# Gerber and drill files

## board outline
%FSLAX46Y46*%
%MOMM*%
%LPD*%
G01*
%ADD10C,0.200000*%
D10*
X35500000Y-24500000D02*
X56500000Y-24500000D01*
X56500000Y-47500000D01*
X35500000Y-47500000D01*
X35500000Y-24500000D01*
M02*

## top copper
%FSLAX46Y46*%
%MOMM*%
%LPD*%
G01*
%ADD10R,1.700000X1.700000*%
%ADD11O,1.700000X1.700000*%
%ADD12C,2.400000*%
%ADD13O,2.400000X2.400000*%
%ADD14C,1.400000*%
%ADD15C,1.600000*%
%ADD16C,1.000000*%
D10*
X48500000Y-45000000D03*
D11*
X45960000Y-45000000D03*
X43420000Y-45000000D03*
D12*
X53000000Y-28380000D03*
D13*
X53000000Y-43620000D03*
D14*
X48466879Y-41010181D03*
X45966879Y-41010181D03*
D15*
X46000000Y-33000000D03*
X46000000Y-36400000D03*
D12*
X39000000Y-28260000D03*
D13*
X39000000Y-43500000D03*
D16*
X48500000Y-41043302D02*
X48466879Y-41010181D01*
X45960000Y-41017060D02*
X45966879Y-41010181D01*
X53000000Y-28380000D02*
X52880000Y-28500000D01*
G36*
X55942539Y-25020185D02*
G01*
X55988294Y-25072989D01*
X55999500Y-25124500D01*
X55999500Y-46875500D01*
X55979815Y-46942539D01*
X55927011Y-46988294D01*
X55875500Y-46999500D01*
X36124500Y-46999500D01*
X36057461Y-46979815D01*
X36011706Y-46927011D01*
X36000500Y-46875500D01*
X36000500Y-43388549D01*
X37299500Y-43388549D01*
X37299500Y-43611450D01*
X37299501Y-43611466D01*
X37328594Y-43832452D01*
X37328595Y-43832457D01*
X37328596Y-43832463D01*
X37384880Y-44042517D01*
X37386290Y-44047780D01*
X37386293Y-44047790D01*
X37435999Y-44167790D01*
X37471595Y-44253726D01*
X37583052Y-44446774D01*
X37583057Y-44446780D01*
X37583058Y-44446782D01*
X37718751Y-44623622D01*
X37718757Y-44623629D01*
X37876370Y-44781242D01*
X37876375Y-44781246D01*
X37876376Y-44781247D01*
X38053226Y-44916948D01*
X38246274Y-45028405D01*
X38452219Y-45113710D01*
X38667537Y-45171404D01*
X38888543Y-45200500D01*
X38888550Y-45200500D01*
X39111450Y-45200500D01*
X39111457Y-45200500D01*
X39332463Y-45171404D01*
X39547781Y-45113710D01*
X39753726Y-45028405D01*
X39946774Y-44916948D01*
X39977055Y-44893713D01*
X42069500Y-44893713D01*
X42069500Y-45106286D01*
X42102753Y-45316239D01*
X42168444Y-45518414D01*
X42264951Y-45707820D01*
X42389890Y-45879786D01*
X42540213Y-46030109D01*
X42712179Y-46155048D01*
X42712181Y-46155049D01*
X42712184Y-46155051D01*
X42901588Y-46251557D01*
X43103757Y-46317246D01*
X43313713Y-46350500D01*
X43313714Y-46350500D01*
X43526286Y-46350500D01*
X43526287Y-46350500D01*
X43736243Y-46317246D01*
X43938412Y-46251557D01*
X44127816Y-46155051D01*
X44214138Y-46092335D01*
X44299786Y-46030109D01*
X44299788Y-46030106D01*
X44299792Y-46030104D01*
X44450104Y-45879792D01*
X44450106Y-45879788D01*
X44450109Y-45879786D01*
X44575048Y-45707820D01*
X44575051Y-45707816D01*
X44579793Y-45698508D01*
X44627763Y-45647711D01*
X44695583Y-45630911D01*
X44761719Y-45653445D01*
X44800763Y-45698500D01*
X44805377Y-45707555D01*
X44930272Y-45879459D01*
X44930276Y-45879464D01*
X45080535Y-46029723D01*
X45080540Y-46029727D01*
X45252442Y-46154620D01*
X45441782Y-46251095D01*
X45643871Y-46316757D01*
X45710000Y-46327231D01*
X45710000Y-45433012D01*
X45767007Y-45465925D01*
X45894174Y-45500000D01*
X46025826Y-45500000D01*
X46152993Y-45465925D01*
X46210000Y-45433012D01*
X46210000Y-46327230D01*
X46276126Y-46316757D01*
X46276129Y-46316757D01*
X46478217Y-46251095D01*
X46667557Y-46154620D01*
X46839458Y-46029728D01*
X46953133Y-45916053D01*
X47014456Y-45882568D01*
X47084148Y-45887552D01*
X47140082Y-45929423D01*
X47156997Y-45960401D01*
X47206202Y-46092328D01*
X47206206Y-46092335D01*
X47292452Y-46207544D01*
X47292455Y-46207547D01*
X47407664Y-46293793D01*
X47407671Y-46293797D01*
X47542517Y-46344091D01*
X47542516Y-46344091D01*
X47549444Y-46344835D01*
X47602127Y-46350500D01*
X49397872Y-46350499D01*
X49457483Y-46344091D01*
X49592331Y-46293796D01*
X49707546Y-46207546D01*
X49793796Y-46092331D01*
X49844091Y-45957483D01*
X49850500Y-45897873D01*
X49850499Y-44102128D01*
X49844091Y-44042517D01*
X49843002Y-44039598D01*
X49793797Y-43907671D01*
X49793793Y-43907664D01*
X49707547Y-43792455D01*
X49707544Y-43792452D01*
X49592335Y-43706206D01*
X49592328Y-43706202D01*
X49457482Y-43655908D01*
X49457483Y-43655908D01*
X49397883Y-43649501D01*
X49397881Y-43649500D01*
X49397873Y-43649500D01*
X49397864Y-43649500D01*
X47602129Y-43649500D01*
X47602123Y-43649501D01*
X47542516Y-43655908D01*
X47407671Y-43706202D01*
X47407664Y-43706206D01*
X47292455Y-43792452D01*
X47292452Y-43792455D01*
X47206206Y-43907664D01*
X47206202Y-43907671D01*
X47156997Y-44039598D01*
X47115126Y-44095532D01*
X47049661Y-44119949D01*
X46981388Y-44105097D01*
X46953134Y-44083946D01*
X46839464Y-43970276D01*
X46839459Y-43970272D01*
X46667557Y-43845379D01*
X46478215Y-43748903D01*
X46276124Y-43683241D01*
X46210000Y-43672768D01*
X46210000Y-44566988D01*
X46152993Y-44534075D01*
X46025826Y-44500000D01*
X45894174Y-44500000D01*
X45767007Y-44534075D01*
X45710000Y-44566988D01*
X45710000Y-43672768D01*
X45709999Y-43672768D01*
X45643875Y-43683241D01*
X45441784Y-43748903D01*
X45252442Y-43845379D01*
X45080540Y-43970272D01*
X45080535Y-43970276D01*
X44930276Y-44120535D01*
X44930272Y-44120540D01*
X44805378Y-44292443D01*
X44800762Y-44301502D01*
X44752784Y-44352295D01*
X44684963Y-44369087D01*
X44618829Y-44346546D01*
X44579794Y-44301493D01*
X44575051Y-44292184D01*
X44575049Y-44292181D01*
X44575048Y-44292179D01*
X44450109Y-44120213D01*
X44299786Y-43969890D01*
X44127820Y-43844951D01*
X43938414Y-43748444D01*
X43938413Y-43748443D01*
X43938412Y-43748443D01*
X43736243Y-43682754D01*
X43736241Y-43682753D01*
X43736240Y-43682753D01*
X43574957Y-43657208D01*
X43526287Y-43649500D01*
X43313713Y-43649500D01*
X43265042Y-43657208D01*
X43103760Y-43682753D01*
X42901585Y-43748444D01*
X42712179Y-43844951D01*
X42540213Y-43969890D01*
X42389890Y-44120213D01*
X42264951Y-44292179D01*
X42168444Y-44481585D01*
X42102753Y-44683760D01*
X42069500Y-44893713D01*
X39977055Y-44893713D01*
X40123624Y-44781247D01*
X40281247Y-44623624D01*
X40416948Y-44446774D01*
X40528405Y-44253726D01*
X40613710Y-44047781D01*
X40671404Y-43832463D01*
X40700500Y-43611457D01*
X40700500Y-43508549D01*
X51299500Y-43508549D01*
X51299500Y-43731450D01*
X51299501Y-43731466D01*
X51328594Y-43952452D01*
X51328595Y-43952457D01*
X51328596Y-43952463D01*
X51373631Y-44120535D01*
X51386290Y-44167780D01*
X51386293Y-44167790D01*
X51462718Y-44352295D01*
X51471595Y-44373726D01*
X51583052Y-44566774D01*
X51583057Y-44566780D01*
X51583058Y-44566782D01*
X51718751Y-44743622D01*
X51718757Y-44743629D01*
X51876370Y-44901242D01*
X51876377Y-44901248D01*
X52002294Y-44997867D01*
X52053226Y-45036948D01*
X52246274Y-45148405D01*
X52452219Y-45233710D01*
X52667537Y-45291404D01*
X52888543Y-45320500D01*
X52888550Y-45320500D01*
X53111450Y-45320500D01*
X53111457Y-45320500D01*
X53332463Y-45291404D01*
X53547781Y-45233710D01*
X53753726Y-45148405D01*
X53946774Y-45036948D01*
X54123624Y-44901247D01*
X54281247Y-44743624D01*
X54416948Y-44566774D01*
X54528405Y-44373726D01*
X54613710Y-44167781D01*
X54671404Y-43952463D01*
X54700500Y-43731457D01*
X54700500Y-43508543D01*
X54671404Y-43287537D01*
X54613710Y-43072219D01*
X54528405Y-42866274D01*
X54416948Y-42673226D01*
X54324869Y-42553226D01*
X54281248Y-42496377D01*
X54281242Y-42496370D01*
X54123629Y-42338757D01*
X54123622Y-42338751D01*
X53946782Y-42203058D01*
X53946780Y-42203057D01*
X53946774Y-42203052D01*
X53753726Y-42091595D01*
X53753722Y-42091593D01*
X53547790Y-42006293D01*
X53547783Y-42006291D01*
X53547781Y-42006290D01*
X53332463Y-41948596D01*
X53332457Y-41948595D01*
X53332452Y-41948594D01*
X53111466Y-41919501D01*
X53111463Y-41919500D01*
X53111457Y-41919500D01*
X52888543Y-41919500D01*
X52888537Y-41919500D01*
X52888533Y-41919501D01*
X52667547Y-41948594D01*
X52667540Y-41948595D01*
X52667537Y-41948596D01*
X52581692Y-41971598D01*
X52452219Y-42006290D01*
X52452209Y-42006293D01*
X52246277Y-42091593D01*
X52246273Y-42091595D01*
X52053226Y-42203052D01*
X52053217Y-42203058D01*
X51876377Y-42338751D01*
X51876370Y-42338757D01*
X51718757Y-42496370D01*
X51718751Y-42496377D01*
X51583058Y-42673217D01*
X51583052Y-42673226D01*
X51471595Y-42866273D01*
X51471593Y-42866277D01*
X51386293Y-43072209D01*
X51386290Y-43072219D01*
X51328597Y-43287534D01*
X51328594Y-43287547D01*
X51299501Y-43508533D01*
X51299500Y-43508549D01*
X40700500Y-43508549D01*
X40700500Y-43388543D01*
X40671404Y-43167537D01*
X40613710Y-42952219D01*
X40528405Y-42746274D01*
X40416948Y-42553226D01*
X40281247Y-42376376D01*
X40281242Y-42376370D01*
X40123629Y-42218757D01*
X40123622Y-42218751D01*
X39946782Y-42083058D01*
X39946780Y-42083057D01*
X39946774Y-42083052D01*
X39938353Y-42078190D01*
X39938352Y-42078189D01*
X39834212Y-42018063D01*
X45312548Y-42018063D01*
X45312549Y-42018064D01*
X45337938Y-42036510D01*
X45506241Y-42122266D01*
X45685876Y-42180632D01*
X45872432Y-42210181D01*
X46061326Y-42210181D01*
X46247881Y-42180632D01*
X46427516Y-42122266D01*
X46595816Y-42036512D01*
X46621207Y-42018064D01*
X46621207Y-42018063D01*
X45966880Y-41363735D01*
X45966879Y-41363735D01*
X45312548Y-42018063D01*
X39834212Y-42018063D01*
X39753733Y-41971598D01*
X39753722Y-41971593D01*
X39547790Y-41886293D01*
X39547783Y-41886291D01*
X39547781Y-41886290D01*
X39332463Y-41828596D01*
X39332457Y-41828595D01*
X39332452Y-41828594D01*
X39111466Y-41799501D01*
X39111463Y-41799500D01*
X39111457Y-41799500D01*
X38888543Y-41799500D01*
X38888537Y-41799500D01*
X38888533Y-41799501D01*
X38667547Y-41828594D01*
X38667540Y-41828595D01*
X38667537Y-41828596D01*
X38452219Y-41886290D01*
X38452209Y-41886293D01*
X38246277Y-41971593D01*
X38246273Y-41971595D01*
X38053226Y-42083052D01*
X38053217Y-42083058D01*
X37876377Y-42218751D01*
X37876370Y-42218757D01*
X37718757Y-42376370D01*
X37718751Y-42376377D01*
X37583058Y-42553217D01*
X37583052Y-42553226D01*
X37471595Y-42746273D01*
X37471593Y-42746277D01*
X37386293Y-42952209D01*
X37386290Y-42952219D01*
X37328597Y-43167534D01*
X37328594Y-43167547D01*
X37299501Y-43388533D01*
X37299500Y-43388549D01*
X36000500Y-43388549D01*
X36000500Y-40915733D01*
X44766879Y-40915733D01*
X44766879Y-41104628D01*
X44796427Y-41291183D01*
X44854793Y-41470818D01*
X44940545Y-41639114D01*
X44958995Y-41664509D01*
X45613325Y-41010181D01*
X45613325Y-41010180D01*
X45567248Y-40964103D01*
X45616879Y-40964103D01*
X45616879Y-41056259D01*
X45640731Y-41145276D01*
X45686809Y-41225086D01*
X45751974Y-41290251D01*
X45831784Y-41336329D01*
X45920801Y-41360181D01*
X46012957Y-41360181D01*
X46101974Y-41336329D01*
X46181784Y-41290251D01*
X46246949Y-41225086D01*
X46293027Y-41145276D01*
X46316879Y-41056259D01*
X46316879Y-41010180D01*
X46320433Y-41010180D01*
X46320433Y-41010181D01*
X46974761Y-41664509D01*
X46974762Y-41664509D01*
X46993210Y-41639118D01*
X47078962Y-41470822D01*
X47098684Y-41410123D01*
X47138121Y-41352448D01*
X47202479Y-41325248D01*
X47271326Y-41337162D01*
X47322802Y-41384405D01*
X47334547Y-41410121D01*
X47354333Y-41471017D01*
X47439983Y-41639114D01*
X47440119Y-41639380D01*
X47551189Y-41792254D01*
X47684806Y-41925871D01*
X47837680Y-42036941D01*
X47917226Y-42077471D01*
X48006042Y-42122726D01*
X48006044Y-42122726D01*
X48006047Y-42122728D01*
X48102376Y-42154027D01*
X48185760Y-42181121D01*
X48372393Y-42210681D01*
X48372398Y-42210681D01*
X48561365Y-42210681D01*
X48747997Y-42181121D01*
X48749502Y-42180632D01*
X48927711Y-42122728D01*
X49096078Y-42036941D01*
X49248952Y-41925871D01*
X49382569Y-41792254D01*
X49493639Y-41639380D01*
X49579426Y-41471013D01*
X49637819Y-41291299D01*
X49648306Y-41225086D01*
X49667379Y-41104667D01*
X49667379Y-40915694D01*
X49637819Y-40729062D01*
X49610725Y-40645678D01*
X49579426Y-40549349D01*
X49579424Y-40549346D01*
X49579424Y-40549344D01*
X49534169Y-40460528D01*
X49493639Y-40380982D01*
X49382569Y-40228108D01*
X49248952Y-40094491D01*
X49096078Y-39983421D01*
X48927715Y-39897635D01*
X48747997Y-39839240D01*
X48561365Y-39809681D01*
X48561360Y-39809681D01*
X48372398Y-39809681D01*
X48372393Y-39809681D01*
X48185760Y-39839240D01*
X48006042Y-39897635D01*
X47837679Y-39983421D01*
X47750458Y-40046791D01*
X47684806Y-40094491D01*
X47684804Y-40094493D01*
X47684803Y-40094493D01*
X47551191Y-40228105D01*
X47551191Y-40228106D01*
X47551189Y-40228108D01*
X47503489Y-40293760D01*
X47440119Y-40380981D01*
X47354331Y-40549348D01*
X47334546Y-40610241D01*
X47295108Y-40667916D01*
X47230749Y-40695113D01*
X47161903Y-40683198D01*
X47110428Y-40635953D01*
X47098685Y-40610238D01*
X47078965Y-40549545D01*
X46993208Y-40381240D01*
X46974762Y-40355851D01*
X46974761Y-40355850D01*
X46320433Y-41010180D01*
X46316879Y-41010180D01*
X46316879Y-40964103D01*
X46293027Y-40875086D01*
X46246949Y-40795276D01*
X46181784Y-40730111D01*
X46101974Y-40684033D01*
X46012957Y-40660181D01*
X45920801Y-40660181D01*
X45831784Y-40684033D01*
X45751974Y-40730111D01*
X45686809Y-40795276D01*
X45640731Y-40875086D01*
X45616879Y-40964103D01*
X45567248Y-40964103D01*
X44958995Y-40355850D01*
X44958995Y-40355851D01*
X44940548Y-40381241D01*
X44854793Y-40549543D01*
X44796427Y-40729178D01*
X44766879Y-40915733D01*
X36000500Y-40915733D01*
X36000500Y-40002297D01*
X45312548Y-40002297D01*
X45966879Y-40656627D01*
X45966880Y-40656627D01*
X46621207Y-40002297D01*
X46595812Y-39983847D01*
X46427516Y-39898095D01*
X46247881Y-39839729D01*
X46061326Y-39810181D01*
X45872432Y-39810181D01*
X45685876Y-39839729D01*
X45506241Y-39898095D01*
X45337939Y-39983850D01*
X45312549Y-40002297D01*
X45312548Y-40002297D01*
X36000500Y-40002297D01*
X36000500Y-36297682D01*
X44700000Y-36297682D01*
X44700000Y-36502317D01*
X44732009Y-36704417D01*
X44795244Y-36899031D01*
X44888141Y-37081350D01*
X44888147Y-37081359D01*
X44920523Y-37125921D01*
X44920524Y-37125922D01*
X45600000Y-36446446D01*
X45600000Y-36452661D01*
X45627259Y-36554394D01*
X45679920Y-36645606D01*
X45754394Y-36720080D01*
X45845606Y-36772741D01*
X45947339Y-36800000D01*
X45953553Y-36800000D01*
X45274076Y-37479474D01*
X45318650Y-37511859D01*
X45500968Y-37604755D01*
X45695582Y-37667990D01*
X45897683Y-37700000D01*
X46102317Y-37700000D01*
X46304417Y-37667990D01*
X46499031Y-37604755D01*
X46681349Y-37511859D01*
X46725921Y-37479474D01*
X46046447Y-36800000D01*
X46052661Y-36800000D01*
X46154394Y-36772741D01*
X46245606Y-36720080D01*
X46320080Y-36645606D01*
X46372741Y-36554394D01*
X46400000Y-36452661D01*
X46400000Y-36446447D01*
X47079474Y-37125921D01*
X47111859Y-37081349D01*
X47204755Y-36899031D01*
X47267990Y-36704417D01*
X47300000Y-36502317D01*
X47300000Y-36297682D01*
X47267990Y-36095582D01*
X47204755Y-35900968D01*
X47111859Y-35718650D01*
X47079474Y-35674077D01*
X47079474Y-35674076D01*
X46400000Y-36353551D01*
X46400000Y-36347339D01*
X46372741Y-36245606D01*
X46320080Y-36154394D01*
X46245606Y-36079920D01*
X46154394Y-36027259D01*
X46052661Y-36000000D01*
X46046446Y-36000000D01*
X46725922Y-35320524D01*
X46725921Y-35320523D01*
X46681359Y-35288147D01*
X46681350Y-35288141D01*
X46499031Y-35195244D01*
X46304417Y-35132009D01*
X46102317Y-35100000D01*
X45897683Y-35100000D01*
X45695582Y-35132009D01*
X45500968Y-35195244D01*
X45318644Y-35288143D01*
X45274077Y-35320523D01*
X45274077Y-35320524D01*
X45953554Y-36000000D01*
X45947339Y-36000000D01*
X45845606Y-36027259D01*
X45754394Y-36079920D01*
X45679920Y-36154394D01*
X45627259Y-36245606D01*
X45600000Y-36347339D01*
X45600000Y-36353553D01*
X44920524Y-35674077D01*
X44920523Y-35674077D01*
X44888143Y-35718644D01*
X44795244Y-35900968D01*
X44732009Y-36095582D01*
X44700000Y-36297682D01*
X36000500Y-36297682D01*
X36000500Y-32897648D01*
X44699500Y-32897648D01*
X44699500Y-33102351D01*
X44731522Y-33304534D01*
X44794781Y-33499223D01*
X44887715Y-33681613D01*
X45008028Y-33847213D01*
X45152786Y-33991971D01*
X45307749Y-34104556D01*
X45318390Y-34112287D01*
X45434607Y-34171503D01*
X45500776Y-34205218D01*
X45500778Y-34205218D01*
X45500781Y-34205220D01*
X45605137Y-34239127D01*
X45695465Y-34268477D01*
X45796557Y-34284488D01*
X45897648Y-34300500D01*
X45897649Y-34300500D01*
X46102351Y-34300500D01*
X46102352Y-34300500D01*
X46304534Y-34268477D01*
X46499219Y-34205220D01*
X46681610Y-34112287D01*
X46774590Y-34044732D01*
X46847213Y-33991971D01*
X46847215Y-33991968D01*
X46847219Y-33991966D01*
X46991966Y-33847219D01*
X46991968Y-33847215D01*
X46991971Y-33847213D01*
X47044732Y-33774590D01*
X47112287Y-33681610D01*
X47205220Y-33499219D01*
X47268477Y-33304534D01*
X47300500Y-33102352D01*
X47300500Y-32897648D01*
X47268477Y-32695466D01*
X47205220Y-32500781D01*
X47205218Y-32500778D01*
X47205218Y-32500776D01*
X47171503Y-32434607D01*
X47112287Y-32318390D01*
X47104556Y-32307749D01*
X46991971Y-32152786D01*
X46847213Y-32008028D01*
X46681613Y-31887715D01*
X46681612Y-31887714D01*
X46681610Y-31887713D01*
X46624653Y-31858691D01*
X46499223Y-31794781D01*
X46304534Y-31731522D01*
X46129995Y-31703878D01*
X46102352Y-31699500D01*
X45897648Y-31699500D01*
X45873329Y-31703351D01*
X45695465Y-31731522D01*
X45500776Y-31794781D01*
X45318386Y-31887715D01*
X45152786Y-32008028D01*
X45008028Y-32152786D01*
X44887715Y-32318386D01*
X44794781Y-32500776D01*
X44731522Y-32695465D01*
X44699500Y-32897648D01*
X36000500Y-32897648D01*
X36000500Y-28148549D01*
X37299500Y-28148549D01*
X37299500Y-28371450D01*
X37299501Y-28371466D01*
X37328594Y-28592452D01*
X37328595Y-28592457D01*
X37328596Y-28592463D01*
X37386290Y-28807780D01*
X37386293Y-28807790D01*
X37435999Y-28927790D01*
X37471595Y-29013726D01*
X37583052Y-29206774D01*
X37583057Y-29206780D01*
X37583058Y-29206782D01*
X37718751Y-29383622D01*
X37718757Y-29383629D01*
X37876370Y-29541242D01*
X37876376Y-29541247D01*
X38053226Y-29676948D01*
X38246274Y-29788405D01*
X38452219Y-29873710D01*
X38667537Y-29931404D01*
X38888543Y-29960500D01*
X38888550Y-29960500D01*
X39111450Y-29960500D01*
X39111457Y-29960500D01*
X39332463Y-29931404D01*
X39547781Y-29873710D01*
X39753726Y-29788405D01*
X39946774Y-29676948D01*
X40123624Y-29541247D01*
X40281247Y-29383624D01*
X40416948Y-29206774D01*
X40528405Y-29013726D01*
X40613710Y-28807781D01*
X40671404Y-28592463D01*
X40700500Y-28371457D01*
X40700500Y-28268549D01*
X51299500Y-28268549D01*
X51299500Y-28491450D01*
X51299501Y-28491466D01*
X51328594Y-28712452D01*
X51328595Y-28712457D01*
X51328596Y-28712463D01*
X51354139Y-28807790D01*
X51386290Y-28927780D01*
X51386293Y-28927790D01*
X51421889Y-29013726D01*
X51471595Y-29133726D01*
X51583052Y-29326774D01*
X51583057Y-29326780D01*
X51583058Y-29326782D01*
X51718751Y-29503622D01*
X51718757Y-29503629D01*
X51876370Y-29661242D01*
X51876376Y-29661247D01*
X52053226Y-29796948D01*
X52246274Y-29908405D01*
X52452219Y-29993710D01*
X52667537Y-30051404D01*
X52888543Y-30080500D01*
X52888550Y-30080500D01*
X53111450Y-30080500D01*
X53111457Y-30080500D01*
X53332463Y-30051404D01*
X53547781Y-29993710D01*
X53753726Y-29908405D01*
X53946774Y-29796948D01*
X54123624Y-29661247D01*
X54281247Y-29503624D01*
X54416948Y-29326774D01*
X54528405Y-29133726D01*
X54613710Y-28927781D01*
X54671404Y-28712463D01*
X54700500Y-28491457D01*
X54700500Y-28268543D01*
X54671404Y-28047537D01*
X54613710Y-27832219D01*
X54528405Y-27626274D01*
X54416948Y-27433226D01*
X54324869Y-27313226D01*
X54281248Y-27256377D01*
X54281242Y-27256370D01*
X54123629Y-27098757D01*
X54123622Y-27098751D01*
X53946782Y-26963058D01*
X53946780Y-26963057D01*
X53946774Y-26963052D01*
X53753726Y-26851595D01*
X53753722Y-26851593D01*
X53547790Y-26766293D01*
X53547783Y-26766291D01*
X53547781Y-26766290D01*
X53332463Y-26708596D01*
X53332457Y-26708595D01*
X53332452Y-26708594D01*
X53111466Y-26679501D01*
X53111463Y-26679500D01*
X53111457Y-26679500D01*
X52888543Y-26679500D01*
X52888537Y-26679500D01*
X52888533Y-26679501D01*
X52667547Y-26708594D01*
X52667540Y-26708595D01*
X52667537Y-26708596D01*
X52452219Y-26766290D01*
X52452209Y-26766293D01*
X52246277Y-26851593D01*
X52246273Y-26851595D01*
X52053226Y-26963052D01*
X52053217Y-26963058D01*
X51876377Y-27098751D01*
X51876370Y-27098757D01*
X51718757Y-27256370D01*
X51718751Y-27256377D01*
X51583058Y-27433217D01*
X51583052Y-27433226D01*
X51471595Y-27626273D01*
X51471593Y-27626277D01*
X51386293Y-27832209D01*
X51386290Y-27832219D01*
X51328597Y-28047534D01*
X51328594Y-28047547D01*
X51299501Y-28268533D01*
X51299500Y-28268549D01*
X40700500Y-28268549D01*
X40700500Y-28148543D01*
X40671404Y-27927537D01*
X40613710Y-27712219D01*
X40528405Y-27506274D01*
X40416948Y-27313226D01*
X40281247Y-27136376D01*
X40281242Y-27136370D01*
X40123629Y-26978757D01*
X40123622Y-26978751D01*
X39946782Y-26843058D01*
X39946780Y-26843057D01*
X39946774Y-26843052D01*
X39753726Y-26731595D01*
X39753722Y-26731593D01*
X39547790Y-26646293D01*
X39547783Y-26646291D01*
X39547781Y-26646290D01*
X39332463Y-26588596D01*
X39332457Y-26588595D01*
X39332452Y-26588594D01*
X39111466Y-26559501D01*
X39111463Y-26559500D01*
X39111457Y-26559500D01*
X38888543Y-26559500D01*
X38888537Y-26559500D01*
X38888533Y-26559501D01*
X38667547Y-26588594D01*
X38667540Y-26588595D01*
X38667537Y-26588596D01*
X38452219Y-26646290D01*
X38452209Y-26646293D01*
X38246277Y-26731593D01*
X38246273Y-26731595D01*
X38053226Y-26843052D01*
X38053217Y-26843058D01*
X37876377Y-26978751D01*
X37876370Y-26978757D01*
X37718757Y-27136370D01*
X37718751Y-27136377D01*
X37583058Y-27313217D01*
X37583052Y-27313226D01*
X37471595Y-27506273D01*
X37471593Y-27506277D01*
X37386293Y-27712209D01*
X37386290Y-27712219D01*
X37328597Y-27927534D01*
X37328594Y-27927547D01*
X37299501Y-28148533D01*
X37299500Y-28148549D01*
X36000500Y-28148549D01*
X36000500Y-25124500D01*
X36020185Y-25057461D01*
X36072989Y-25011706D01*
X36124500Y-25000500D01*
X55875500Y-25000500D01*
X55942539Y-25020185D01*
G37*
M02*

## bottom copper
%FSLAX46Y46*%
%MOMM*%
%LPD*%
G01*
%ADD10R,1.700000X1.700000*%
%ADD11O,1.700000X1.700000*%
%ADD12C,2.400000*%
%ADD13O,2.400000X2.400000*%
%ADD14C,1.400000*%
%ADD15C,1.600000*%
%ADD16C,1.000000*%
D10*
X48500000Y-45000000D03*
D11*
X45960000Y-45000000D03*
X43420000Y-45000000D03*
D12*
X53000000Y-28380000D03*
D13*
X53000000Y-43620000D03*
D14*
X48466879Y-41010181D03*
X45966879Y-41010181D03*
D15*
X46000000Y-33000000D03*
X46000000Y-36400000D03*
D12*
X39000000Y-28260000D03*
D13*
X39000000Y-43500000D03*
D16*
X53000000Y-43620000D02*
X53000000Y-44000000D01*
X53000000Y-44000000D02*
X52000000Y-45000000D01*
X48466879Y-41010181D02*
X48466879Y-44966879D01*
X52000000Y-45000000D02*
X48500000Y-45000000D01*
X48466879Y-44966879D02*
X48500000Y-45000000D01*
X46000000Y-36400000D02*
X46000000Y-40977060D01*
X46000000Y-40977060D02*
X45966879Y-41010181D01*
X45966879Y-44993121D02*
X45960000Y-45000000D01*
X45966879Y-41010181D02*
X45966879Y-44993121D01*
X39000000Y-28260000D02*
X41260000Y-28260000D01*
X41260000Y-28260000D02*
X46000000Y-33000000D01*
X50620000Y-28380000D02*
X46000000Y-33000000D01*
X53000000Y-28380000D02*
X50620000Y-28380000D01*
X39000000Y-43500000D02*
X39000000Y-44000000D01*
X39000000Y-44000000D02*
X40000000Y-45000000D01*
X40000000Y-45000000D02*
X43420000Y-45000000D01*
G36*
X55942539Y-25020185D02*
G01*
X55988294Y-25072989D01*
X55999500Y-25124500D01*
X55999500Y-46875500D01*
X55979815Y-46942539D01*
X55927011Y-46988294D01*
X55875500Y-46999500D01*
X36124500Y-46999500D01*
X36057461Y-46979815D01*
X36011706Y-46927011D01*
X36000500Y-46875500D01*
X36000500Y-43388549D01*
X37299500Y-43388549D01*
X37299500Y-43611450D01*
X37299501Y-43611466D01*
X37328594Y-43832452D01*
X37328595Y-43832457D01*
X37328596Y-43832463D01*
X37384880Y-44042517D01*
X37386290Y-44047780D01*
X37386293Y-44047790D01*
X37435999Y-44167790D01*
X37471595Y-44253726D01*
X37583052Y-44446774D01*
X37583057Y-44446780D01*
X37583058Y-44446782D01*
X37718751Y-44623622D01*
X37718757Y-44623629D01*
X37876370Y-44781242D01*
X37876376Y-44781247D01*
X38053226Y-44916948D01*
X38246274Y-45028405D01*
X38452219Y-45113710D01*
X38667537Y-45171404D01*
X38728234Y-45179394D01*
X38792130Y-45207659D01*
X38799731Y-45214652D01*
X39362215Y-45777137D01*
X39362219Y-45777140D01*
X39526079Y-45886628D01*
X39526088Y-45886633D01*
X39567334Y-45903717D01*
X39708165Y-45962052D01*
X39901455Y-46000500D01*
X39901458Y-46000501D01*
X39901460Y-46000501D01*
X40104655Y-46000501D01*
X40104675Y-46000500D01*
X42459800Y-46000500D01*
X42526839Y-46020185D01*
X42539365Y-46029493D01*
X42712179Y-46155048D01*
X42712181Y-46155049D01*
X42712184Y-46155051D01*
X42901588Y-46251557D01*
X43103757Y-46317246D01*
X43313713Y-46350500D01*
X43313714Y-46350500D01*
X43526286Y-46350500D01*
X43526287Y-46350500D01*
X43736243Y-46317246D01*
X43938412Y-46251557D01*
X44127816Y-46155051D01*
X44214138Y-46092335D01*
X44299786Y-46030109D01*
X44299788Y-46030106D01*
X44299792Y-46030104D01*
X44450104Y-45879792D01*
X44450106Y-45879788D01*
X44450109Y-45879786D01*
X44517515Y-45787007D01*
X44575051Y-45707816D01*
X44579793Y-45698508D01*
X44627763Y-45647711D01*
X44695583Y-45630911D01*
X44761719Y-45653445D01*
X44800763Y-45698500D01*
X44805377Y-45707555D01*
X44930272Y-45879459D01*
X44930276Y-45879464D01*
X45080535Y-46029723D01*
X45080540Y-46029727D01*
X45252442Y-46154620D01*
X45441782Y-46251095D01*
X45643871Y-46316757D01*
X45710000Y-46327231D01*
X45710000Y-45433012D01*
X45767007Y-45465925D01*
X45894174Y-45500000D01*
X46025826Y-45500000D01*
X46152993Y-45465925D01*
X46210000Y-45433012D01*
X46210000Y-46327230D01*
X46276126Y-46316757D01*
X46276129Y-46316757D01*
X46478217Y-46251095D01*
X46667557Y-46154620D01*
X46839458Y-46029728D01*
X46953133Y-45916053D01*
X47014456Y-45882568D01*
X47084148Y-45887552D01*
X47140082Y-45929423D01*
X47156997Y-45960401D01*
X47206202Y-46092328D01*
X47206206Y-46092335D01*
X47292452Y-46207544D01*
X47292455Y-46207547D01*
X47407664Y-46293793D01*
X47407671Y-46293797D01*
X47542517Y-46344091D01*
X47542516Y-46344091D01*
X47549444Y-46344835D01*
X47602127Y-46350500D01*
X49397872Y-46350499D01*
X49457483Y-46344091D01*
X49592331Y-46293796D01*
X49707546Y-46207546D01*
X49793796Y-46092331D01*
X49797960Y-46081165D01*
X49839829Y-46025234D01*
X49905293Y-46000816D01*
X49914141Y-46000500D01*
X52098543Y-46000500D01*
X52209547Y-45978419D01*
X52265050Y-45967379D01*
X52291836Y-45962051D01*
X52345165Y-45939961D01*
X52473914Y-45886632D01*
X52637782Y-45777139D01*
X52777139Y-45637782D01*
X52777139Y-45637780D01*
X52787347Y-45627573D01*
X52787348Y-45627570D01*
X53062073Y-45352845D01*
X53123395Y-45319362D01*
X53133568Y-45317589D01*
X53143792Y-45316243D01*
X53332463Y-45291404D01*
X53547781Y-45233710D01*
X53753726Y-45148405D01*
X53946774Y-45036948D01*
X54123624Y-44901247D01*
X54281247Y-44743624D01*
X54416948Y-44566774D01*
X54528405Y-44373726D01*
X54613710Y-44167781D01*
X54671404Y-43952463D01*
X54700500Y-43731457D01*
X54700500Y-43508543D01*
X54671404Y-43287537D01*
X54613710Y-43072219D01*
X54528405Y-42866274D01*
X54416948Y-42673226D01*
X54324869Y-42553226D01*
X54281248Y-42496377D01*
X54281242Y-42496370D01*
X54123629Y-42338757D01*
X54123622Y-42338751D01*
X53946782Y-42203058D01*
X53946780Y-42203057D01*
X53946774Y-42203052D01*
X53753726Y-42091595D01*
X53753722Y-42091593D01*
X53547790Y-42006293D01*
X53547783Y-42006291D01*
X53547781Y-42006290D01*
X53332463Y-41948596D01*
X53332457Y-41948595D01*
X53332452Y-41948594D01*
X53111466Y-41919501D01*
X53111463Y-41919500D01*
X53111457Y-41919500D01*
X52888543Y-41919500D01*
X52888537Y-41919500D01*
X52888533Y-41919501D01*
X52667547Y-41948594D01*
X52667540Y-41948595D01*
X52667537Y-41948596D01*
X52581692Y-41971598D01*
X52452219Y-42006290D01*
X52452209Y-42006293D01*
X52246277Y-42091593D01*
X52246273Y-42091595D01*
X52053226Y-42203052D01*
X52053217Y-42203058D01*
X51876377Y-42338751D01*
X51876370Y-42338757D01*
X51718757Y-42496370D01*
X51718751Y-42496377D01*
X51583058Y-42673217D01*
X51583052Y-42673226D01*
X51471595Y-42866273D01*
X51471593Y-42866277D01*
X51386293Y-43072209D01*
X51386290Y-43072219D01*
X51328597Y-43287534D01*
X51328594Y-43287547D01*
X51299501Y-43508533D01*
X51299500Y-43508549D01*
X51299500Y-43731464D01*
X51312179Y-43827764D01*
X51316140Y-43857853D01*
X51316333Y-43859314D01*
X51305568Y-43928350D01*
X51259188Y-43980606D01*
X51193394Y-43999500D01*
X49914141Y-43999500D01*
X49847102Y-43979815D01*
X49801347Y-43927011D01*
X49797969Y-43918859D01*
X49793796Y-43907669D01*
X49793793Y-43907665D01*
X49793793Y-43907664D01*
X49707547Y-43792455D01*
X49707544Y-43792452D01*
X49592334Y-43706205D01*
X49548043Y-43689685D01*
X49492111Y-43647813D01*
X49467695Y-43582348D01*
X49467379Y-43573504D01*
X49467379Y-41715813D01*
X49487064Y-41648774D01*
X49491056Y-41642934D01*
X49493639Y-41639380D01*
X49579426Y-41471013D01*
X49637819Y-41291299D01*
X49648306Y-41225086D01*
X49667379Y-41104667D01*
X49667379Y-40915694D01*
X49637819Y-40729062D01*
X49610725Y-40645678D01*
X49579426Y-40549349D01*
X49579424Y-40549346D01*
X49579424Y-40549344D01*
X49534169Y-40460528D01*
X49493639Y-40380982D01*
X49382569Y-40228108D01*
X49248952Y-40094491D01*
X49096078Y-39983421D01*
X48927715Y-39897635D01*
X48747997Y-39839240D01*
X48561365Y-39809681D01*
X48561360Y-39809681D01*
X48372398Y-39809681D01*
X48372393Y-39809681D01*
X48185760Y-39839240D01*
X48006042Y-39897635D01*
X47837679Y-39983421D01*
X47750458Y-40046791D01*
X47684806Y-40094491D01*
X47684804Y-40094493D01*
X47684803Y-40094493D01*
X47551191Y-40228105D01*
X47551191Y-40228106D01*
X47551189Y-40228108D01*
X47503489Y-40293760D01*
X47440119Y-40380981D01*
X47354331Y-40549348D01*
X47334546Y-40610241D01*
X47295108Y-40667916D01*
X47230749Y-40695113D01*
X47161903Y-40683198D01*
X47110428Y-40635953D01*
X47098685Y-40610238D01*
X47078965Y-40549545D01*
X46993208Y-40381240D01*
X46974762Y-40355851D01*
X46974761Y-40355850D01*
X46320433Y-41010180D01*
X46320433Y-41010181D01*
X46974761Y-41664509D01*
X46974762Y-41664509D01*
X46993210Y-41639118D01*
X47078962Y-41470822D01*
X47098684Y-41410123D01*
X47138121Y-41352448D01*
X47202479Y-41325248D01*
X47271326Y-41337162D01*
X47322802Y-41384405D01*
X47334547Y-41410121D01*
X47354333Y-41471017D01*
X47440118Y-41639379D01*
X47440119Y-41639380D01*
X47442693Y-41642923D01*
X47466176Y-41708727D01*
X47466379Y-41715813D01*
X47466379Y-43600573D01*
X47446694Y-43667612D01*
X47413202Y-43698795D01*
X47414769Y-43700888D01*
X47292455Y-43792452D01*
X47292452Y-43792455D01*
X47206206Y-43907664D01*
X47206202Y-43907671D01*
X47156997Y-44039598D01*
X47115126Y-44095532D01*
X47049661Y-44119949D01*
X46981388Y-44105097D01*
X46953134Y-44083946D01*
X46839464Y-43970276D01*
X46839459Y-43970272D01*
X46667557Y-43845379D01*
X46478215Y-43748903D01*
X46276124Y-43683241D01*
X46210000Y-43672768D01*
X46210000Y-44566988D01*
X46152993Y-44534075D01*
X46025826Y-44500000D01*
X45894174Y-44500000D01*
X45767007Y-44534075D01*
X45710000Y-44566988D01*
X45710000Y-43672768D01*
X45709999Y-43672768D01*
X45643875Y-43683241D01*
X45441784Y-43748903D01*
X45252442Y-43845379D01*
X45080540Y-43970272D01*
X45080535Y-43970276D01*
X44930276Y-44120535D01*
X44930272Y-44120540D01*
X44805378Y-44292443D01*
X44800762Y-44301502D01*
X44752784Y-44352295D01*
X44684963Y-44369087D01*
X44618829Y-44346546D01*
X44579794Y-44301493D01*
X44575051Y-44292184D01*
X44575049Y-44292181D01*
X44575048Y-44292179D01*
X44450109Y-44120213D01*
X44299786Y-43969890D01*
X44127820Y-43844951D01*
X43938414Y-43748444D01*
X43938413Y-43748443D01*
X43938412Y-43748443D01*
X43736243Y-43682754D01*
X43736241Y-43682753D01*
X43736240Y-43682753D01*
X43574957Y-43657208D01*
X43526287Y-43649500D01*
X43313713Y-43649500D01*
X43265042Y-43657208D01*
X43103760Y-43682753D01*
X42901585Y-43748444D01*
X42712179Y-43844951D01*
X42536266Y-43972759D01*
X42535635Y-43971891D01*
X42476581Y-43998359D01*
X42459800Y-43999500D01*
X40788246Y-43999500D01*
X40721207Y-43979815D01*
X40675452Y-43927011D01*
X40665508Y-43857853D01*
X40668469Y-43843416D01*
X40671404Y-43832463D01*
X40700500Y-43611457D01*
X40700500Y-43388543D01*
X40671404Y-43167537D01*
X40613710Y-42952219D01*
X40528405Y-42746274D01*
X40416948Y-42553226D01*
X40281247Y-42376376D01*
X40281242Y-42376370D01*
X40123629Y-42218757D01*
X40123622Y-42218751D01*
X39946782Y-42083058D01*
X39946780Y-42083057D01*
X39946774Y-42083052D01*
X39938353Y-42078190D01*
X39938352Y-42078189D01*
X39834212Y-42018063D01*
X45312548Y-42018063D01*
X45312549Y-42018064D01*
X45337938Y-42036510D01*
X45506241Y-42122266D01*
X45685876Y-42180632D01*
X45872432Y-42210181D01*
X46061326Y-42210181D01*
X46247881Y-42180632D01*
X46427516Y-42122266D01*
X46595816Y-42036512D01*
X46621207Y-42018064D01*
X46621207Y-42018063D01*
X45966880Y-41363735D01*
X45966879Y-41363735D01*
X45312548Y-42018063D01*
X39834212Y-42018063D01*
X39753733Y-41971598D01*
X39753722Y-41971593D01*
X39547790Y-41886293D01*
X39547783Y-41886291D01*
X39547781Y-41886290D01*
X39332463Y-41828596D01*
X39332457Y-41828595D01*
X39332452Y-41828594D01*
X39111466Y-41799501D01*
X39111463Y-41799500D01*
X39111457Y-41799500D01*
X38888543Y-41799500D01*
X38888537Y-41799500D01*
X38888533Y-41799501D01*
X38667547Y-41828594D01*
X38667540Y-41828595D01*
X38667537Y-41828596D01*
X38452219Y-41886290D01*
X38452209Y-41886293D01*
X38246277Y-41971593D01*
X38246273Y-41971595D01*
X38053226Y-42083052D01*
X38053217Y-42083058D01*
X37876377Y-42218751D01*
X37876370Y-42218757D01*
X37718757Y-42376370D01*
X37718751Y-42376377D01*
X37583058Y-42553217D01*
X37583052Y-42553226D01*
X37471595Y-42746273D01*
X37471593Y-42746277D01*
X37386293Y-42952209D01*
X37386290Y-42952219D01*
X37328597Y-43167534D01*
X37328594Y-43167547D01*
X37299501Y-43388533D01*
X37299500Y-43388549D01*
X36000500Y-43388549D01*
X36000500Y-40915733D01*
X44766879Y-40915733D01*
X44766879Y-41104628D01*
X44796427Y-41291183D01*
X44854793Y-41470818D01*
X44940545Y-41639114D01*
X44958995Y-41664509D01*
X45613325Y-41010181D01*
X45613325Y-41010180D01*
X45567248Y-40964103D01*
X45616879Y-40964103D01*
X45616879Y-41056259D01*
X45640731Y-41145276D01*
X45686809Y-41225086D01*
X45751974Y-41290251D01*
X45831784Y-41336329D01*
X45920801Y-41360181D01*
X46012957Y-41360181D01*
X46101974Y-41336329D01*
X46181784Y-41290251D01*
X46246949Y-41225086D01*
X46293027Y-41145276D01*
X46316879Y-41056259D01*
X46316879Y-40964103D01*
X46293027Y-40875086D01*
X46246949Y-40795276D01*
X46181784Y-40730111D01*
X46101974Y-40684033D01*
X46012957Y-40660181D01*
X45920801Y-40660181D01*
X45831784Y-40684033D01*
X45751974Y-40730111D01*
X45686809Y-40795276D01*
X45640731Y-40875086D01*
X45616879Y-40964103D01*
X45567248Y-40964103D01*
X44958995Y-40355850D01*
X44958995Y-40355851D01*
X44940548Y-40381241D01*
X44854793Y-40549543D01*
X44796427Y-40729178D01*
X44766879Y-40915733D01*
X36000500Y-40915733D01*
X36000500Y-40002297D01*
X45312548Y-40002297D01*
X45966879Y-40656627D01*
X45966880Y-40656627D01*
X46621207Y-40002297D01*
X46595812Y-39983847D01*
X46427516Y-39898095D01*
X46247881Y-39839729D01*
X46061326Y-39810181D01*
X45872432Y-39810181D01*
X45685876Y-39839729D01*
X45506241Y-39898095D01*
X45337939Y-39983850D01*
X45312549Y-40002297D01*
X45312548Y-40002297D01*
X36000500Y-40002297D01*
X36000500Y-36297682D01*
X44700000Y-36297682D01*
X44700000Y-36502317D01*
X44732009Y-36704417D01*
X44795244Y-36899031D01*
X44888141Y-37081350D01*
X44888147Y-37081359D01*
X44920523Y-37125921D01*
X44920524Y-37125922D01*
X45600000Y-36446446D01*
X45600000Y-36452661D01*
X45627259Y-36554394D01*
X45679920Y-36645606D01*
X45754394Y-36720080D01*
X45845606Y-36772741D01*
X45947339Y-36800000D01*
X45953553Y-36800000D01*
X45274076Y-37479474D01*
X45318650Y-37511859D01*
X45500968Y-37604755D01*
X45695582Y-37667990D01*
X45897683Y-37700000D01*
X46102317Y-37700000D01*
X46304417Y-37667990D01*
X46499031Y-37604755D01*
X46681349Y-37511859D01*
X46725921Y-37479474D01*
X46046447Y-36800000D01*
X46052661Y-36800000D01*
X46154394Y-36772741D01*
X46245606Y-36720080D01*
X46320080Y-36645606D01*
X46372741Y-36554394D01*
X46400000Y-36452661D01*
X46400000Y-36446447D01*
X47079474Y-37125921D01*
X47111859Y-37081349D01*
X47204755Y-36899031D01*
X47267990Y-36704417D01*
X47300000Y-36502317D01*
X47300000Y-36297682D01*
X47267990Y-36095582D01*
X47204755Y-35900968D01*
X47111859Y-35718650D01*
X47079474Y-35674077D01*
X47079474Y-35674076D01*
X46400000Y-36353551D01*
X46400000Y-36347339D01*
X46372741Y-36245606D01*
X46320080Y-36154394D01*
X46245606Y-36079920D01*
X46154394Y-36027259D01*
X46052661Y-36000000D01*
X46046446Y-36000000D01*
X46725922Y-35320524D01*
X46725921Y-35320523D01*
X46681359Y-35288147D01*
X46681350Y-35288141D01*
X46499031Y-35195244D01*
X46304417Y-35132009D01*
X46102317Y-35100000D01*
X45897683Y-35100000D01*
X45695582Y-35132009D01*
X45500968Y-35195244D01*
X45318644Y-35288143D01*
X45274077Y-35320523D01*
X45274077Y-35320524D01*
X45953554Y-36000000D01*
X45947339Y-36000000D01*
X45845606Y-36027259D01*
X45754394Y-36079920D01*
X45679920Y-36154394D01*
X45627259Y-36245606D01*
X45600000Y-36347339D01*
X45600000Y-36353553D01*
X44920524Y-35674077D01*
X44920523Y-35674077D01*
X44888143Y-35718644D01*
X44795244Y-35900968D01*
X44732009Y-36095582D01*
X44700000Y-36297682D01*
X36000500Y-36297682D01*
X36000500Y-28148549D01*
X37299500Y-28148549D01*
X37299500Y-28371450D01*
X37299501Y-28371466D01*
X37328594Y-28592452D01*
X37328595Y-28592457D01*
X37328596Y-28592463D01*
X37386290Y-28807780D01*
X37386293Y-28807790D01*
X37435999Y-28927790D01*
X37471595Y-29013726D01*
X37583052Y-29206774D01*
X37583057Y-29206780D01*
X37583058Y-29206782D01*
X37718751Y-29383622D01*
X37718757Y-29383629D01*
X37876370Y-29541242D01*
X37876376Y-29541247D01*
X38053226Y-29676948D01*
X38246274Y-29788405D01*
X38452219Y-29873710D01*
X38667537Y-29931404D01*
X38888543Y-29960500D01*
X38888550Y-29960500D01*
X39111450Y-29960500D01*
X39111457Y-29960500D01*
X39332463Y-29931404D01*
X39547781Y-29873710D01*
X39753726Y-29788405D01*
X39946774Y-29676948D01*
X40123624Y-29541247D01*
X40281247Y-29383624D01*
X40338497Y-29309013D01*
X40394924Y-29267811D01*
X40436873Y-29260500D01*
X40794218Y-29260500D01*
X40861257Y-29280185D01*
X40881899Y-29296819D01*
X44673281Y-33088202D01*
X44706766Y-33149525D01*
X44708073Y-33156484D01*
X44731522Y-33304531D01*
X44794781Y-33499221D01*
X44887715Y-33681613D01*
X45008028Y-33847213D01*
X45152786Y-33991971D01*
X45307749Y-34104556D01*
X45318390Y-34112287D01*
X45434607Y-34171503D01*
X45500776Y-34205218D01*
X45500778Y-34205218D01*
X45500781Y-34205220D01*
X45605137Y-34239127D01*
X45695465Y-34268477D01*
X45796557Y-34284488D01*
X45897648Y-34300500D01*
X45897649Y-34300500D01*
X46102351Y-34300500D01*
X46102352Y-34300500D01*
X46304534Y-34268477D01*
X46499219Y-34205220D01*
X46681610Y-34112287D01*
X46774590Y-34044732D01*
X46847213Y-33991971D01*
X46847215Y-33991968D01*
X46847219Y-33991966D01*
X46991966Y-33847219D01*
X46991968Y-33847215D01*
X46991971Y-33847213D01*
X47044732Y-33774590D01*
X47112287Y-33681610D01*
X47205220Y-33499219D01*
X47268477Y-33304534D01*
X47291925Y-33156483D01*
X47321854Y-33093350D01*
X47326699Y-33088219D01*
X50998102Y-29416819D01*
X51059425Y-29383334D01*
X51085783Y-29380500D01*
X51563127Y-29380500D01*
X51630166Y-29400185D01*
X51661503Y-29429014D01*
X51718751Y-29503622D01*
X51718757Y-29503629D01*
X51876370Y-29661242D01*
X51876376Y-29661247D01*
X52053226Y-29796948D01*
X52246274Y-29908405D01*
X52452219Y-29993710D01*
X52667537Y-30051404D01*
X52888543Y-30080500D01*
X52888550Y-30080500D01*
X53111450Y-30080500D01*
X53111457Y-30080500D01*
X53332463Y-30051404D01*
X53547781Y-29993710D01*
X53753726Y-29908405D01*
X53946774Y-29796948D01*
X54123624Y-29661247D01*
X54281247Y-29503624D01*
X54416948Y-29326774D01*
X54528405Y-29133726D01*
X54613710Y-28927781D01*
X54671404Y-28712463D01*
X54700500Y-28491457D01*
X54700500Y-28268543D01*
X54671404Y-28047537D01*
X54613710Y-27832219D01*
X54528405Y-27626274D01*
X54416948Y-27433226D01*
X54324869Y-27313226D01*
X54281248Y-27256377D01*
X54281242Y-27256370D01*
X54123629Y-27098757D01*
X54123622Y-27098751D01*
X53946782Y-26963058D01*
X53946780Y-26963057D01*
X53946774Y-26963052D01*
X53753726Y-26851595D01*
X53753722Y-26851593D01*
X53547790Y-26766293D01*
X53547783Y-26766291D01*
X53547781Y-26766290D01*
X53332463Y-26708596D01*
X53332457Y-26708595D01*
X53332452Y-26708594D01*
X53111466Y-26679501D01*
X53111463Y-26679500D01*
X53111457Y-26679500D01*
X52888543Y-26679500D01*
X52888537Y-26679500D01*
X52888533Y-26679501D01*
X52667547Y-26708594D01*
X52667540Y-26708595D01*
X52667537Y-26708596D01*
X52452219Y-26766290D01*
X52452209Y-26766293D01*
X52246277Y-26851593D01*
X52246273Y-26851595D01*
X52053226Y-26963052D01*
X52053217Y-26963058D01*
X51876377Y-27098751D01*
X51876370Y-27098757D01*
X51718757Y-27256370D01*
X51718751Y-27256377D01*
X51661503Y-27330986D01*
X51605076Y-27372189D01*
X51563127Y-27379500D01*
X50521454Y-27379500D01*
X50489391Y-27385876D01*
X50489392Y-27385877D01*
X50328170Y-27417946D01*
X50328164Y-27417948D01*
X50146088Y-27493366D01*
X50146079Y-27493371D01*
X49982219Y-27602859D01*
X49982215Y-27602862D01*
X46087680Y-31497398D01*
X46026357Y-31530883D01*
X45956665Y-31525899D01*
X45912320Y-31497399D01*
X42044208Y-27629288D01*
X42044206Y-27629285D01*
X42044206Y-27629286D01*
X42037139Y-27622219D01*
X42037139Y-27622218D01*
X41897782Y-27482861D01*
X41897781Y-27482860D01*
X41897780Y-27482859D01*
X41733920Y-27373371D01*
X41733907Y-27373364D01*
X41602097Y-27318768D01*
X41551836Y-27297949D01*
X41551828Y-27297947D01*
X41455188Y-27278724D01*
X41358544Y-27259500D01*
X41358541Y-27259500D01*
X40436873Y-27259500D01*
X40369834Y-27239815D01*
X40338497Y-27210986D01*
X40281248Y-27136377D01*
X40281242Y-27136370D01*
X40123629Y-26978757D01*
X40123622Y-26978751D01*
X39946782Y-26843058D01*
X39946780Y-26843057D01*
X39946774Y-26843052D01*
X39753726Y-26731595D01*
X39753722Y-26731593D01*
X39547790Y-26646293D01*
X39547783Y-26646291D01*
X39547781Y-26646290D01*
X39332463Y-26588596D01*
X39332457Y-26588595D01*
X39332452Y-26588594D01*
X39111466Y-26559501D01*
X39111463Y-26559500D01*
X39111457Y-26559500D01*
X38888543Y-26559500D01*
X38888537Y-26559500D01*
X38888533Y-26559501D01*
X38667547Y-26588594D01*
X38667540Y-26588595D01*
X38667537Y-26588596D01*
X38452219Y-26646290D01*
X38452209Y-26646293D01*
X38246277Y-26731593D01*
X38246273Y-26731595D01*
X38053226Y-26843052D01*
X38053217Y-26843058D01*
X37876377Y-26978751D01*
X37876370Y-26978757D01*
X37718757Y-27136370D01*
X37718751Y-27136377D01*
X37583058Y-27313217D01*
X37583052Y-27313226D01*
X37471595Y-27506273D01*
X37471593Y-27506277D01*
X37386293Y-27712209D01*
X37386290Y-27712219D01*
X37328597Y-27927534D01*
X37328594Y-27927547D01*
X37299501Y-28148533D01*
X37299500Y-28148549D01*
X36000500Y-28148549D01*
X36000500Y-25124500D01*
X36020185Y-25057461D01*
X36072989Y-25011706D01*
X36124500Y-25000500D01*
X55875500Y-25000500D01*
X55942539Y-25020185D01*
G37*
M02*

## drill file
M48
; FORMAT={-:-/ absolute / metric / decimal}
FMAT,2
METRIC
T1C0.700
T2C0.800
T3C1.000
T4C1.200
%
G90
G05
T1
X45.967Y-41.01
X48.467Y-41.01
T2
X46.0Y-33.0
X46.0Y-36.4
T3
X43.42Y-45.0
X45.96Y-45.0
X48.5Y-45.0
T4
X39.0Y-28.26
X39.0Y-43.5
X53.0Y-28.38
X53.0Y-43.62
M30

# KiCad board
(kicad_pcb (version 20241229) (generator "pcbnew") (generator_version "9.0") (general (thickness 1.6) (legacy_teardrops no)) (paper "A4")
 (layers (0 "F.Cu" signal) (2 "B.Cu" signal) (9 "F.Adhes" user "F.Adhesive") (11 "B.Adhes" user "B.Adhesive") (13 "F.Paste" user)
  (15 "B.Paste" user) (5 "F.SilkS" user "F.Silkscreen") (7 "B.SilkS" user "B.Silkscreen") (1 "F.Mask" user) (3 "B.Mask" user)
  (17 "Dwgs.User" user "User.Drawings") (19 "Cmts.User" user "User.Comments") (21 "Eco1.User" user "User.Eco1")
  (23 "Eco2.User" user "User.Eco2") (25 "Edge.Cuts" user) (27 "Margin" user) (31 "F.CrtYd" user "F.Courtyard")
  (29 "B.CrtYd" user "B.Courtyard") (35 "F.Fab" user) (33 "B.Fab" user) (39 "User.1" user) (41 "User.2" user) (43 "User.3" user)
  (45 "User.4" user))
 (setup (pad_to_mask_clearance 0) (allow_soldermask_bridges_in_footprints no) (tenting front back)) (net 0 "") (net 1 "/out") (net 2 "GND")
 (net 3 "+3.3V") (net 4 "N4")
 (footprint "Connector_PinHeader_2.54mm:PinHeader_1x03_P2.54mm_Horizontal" (layer "F.Cu") (at 48.5 45 -90)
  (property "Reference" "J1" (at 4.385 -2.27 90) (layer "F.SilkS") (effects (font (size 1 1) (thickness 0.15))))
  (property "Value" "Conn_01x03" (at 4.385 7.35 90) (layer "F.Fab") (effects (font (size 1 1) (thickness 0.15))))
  (pad "1" thru_hole rect (at 0 0 270) (size 1.7 1.7) (drill 1) (layers "*.Cu" "*.Mask") (remove_unused_layers no) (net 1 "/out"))
  (pad "2" thru_hole oval (at 0 2.54 270) (size 1.7 1.7) (drill 1) (layers "*.Cu" "*.Mask") (remove_unused_layers no) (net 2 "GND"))
  (pad "3" thru_hole oval (at 0 5.08 270) (size 1.7 1.7) (drill 1) (layers "*.Cu" "*.Mask") (remove_unused_layers no) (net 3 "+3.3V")))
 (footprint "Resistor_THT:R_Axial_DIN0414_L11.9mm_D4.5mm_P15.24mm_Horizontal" (layer "F.Cu") (at 53 28.38 -90)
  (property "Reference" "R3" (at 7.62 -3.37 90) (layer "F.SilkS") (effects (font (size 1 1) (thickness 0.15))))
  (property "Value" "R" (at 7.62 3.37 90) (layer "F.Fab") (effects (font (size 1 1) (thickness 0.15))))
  (pad "1" thru_hole circle (at 0 0 270) (size 2.4 2.4) (drill 1.2) (layers "*.Cu" "*.Mask") (remove_unused_layers no) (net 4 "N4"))
  (pad "2" thru_hole oval (at 15.24 0 270) (size 2.4 2.4) (drill 1.2) (layers "*.Cu" "*.Mask") (remove_unused_layers no) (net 1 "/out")))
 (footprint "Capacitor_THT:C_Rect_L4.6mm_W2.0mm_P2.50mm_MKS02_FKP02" (layer "F.Cu") (at 48.466879 41.010181 180)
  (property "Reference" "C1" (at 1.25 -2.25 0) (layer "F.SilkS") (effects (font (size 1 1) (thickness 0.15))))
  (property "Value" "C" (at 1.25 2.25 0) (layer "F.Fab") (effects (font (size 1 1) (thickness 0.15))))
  (pad "1" thru_hole circle (at 0 0 180) (size 1.4 1.4) (drill 0.7) (layers "*.Cu" "*.Mask") (remove_unused_layers no) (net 1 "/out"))
  (pad "2" thru_hole circle (at 2.5 0 180) (size 1.4 1.4) (drill 0.7) (layers "*.Cu" "*.Mask") (remove_unused_layers no) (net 2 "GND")))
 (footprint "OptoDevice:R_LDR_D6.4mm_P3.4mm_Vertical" (layer "F.Cu") (at 46 33 -90)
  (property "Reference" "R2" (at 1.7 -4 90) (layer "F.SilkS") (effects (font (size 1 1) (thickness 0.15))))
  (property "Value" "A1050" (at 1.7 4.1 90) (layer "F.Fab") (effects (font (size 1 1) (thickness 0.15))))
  (pad "1" thru_hole circle (at 0 0 270) (size 1.6 1.6) (drill 0.8) (layers "*.Cu" "*.Mask") (remove_unused_layers no) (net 4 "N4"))
  (pad "2" thru_hole circle (at 3.4 0 270) (size 1.6 1.6) (drill 0.8) (layers "*.Cu" "*.Mask") (remove_unused_layers no) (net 2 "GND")))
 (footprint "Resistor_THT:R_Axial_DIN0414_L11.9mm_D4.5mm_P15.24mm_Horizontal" (layer "F.Cu") (at 39 28.26 -90)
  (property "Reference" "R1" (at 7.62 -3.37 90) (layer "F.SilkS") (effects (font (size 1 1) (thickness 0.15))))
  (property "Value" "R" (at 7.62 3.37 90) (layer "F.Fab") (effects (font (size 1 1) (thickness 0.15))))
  (pad "1" thru_hole circle (at 0 0 270) (size 2.4 2.4) (drill 1.2) (layers "*.Cu" "*.Mask") (remove_unused_layers no) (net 4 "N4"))
  (pad "2" thru_hole oval (at 15.24 0 270) (size 2.4 2.4) (drill 1.2) (layers "*.Cu" "*.Mask") (remove_unused_layers no) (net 3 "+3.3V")))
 (gr_rect (start 35.5 24.5) (end 56.5 47.5) (stroke (width 0.2) (type solid)) (fill no) (layer "Edge.Cuts"))
 (segment (start 48.5 41.043302) (end 48.466879 41.010181) (width 1) (layer "F.Cu") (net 1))
 (segment (start 53 43.62) (end 53 44) (width 1) (layer "B.Cu") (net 1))
 (segment (start 53 44) (end 52 45) (width 1) (layer "B.Cu") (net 1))
 (segment (start 48.466879 41.010181) (end 48.466879 44.966879) (width 1) (layer "B.Cu") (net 1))
 (segment (start 52 45) (end 48.5 45) (width 1) (layer "B.Cu") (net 1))
 (segment (start 48.466879 44.966879) (end 48.5 45) (width 1) (layer "B.Cu") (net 1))
 (segment (start 45.96 41.01706) (end 45.966879 41.010181) (width 1) (layer "F.Cu") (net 2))
 (segment (start 46 36.4) (end 46 40.97706) (width 1) (layer "B.Cu") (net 2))
 (segment (start 46 40.97706) (end 45.966879 41.010181) (width 1) (layer "B.Cu") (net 2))
 (segment (start 45.966879 44.993121) (end 45.96 45) (width 1) (layer "B.Cu") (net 2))
 (segment (start 45.966879 41.010181) (end 45.966879 44.993121) (width 1) (layer "B.Cu") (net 2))
 (segment (start 53 28.38) (end 52.88 28.5) (width 1) (layer "F.Cu") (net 4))
 (segment (start 39 28.26) (end 41.26 28.26) (width 1) (layer "B.Cu") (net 4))
 (segment (start 41.26 28.26) (end 46 33) (width 1) (layer "B.Cu") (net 4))
 (segment (start 50.62 28.38) (end 46 33) (width 1) (layer "B.Cu") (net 4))
 (segment (start 53 28.38) (end 50.62 28.38) (width 1) (layer "B.Cu") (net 4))
 (segment (start 39 43.5) (end 39 44) (width 1) (layer "B.Cu") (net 3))
 (segment (start 39 44) (end 40 45) (width 1) (layer "B.Cu") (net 3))
 (segment (start 40 45) (end 43.42 45) (width 1) (layer "B.Cu") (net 3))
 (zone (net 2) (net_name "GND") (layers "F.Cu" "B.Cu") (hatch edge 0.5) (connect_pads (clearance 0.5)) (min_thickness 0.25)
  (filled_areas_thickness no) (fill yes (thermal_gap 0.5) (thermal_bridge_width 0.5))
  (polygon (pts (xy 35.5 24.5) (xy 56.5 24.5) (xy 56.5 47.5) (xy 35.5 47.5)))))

